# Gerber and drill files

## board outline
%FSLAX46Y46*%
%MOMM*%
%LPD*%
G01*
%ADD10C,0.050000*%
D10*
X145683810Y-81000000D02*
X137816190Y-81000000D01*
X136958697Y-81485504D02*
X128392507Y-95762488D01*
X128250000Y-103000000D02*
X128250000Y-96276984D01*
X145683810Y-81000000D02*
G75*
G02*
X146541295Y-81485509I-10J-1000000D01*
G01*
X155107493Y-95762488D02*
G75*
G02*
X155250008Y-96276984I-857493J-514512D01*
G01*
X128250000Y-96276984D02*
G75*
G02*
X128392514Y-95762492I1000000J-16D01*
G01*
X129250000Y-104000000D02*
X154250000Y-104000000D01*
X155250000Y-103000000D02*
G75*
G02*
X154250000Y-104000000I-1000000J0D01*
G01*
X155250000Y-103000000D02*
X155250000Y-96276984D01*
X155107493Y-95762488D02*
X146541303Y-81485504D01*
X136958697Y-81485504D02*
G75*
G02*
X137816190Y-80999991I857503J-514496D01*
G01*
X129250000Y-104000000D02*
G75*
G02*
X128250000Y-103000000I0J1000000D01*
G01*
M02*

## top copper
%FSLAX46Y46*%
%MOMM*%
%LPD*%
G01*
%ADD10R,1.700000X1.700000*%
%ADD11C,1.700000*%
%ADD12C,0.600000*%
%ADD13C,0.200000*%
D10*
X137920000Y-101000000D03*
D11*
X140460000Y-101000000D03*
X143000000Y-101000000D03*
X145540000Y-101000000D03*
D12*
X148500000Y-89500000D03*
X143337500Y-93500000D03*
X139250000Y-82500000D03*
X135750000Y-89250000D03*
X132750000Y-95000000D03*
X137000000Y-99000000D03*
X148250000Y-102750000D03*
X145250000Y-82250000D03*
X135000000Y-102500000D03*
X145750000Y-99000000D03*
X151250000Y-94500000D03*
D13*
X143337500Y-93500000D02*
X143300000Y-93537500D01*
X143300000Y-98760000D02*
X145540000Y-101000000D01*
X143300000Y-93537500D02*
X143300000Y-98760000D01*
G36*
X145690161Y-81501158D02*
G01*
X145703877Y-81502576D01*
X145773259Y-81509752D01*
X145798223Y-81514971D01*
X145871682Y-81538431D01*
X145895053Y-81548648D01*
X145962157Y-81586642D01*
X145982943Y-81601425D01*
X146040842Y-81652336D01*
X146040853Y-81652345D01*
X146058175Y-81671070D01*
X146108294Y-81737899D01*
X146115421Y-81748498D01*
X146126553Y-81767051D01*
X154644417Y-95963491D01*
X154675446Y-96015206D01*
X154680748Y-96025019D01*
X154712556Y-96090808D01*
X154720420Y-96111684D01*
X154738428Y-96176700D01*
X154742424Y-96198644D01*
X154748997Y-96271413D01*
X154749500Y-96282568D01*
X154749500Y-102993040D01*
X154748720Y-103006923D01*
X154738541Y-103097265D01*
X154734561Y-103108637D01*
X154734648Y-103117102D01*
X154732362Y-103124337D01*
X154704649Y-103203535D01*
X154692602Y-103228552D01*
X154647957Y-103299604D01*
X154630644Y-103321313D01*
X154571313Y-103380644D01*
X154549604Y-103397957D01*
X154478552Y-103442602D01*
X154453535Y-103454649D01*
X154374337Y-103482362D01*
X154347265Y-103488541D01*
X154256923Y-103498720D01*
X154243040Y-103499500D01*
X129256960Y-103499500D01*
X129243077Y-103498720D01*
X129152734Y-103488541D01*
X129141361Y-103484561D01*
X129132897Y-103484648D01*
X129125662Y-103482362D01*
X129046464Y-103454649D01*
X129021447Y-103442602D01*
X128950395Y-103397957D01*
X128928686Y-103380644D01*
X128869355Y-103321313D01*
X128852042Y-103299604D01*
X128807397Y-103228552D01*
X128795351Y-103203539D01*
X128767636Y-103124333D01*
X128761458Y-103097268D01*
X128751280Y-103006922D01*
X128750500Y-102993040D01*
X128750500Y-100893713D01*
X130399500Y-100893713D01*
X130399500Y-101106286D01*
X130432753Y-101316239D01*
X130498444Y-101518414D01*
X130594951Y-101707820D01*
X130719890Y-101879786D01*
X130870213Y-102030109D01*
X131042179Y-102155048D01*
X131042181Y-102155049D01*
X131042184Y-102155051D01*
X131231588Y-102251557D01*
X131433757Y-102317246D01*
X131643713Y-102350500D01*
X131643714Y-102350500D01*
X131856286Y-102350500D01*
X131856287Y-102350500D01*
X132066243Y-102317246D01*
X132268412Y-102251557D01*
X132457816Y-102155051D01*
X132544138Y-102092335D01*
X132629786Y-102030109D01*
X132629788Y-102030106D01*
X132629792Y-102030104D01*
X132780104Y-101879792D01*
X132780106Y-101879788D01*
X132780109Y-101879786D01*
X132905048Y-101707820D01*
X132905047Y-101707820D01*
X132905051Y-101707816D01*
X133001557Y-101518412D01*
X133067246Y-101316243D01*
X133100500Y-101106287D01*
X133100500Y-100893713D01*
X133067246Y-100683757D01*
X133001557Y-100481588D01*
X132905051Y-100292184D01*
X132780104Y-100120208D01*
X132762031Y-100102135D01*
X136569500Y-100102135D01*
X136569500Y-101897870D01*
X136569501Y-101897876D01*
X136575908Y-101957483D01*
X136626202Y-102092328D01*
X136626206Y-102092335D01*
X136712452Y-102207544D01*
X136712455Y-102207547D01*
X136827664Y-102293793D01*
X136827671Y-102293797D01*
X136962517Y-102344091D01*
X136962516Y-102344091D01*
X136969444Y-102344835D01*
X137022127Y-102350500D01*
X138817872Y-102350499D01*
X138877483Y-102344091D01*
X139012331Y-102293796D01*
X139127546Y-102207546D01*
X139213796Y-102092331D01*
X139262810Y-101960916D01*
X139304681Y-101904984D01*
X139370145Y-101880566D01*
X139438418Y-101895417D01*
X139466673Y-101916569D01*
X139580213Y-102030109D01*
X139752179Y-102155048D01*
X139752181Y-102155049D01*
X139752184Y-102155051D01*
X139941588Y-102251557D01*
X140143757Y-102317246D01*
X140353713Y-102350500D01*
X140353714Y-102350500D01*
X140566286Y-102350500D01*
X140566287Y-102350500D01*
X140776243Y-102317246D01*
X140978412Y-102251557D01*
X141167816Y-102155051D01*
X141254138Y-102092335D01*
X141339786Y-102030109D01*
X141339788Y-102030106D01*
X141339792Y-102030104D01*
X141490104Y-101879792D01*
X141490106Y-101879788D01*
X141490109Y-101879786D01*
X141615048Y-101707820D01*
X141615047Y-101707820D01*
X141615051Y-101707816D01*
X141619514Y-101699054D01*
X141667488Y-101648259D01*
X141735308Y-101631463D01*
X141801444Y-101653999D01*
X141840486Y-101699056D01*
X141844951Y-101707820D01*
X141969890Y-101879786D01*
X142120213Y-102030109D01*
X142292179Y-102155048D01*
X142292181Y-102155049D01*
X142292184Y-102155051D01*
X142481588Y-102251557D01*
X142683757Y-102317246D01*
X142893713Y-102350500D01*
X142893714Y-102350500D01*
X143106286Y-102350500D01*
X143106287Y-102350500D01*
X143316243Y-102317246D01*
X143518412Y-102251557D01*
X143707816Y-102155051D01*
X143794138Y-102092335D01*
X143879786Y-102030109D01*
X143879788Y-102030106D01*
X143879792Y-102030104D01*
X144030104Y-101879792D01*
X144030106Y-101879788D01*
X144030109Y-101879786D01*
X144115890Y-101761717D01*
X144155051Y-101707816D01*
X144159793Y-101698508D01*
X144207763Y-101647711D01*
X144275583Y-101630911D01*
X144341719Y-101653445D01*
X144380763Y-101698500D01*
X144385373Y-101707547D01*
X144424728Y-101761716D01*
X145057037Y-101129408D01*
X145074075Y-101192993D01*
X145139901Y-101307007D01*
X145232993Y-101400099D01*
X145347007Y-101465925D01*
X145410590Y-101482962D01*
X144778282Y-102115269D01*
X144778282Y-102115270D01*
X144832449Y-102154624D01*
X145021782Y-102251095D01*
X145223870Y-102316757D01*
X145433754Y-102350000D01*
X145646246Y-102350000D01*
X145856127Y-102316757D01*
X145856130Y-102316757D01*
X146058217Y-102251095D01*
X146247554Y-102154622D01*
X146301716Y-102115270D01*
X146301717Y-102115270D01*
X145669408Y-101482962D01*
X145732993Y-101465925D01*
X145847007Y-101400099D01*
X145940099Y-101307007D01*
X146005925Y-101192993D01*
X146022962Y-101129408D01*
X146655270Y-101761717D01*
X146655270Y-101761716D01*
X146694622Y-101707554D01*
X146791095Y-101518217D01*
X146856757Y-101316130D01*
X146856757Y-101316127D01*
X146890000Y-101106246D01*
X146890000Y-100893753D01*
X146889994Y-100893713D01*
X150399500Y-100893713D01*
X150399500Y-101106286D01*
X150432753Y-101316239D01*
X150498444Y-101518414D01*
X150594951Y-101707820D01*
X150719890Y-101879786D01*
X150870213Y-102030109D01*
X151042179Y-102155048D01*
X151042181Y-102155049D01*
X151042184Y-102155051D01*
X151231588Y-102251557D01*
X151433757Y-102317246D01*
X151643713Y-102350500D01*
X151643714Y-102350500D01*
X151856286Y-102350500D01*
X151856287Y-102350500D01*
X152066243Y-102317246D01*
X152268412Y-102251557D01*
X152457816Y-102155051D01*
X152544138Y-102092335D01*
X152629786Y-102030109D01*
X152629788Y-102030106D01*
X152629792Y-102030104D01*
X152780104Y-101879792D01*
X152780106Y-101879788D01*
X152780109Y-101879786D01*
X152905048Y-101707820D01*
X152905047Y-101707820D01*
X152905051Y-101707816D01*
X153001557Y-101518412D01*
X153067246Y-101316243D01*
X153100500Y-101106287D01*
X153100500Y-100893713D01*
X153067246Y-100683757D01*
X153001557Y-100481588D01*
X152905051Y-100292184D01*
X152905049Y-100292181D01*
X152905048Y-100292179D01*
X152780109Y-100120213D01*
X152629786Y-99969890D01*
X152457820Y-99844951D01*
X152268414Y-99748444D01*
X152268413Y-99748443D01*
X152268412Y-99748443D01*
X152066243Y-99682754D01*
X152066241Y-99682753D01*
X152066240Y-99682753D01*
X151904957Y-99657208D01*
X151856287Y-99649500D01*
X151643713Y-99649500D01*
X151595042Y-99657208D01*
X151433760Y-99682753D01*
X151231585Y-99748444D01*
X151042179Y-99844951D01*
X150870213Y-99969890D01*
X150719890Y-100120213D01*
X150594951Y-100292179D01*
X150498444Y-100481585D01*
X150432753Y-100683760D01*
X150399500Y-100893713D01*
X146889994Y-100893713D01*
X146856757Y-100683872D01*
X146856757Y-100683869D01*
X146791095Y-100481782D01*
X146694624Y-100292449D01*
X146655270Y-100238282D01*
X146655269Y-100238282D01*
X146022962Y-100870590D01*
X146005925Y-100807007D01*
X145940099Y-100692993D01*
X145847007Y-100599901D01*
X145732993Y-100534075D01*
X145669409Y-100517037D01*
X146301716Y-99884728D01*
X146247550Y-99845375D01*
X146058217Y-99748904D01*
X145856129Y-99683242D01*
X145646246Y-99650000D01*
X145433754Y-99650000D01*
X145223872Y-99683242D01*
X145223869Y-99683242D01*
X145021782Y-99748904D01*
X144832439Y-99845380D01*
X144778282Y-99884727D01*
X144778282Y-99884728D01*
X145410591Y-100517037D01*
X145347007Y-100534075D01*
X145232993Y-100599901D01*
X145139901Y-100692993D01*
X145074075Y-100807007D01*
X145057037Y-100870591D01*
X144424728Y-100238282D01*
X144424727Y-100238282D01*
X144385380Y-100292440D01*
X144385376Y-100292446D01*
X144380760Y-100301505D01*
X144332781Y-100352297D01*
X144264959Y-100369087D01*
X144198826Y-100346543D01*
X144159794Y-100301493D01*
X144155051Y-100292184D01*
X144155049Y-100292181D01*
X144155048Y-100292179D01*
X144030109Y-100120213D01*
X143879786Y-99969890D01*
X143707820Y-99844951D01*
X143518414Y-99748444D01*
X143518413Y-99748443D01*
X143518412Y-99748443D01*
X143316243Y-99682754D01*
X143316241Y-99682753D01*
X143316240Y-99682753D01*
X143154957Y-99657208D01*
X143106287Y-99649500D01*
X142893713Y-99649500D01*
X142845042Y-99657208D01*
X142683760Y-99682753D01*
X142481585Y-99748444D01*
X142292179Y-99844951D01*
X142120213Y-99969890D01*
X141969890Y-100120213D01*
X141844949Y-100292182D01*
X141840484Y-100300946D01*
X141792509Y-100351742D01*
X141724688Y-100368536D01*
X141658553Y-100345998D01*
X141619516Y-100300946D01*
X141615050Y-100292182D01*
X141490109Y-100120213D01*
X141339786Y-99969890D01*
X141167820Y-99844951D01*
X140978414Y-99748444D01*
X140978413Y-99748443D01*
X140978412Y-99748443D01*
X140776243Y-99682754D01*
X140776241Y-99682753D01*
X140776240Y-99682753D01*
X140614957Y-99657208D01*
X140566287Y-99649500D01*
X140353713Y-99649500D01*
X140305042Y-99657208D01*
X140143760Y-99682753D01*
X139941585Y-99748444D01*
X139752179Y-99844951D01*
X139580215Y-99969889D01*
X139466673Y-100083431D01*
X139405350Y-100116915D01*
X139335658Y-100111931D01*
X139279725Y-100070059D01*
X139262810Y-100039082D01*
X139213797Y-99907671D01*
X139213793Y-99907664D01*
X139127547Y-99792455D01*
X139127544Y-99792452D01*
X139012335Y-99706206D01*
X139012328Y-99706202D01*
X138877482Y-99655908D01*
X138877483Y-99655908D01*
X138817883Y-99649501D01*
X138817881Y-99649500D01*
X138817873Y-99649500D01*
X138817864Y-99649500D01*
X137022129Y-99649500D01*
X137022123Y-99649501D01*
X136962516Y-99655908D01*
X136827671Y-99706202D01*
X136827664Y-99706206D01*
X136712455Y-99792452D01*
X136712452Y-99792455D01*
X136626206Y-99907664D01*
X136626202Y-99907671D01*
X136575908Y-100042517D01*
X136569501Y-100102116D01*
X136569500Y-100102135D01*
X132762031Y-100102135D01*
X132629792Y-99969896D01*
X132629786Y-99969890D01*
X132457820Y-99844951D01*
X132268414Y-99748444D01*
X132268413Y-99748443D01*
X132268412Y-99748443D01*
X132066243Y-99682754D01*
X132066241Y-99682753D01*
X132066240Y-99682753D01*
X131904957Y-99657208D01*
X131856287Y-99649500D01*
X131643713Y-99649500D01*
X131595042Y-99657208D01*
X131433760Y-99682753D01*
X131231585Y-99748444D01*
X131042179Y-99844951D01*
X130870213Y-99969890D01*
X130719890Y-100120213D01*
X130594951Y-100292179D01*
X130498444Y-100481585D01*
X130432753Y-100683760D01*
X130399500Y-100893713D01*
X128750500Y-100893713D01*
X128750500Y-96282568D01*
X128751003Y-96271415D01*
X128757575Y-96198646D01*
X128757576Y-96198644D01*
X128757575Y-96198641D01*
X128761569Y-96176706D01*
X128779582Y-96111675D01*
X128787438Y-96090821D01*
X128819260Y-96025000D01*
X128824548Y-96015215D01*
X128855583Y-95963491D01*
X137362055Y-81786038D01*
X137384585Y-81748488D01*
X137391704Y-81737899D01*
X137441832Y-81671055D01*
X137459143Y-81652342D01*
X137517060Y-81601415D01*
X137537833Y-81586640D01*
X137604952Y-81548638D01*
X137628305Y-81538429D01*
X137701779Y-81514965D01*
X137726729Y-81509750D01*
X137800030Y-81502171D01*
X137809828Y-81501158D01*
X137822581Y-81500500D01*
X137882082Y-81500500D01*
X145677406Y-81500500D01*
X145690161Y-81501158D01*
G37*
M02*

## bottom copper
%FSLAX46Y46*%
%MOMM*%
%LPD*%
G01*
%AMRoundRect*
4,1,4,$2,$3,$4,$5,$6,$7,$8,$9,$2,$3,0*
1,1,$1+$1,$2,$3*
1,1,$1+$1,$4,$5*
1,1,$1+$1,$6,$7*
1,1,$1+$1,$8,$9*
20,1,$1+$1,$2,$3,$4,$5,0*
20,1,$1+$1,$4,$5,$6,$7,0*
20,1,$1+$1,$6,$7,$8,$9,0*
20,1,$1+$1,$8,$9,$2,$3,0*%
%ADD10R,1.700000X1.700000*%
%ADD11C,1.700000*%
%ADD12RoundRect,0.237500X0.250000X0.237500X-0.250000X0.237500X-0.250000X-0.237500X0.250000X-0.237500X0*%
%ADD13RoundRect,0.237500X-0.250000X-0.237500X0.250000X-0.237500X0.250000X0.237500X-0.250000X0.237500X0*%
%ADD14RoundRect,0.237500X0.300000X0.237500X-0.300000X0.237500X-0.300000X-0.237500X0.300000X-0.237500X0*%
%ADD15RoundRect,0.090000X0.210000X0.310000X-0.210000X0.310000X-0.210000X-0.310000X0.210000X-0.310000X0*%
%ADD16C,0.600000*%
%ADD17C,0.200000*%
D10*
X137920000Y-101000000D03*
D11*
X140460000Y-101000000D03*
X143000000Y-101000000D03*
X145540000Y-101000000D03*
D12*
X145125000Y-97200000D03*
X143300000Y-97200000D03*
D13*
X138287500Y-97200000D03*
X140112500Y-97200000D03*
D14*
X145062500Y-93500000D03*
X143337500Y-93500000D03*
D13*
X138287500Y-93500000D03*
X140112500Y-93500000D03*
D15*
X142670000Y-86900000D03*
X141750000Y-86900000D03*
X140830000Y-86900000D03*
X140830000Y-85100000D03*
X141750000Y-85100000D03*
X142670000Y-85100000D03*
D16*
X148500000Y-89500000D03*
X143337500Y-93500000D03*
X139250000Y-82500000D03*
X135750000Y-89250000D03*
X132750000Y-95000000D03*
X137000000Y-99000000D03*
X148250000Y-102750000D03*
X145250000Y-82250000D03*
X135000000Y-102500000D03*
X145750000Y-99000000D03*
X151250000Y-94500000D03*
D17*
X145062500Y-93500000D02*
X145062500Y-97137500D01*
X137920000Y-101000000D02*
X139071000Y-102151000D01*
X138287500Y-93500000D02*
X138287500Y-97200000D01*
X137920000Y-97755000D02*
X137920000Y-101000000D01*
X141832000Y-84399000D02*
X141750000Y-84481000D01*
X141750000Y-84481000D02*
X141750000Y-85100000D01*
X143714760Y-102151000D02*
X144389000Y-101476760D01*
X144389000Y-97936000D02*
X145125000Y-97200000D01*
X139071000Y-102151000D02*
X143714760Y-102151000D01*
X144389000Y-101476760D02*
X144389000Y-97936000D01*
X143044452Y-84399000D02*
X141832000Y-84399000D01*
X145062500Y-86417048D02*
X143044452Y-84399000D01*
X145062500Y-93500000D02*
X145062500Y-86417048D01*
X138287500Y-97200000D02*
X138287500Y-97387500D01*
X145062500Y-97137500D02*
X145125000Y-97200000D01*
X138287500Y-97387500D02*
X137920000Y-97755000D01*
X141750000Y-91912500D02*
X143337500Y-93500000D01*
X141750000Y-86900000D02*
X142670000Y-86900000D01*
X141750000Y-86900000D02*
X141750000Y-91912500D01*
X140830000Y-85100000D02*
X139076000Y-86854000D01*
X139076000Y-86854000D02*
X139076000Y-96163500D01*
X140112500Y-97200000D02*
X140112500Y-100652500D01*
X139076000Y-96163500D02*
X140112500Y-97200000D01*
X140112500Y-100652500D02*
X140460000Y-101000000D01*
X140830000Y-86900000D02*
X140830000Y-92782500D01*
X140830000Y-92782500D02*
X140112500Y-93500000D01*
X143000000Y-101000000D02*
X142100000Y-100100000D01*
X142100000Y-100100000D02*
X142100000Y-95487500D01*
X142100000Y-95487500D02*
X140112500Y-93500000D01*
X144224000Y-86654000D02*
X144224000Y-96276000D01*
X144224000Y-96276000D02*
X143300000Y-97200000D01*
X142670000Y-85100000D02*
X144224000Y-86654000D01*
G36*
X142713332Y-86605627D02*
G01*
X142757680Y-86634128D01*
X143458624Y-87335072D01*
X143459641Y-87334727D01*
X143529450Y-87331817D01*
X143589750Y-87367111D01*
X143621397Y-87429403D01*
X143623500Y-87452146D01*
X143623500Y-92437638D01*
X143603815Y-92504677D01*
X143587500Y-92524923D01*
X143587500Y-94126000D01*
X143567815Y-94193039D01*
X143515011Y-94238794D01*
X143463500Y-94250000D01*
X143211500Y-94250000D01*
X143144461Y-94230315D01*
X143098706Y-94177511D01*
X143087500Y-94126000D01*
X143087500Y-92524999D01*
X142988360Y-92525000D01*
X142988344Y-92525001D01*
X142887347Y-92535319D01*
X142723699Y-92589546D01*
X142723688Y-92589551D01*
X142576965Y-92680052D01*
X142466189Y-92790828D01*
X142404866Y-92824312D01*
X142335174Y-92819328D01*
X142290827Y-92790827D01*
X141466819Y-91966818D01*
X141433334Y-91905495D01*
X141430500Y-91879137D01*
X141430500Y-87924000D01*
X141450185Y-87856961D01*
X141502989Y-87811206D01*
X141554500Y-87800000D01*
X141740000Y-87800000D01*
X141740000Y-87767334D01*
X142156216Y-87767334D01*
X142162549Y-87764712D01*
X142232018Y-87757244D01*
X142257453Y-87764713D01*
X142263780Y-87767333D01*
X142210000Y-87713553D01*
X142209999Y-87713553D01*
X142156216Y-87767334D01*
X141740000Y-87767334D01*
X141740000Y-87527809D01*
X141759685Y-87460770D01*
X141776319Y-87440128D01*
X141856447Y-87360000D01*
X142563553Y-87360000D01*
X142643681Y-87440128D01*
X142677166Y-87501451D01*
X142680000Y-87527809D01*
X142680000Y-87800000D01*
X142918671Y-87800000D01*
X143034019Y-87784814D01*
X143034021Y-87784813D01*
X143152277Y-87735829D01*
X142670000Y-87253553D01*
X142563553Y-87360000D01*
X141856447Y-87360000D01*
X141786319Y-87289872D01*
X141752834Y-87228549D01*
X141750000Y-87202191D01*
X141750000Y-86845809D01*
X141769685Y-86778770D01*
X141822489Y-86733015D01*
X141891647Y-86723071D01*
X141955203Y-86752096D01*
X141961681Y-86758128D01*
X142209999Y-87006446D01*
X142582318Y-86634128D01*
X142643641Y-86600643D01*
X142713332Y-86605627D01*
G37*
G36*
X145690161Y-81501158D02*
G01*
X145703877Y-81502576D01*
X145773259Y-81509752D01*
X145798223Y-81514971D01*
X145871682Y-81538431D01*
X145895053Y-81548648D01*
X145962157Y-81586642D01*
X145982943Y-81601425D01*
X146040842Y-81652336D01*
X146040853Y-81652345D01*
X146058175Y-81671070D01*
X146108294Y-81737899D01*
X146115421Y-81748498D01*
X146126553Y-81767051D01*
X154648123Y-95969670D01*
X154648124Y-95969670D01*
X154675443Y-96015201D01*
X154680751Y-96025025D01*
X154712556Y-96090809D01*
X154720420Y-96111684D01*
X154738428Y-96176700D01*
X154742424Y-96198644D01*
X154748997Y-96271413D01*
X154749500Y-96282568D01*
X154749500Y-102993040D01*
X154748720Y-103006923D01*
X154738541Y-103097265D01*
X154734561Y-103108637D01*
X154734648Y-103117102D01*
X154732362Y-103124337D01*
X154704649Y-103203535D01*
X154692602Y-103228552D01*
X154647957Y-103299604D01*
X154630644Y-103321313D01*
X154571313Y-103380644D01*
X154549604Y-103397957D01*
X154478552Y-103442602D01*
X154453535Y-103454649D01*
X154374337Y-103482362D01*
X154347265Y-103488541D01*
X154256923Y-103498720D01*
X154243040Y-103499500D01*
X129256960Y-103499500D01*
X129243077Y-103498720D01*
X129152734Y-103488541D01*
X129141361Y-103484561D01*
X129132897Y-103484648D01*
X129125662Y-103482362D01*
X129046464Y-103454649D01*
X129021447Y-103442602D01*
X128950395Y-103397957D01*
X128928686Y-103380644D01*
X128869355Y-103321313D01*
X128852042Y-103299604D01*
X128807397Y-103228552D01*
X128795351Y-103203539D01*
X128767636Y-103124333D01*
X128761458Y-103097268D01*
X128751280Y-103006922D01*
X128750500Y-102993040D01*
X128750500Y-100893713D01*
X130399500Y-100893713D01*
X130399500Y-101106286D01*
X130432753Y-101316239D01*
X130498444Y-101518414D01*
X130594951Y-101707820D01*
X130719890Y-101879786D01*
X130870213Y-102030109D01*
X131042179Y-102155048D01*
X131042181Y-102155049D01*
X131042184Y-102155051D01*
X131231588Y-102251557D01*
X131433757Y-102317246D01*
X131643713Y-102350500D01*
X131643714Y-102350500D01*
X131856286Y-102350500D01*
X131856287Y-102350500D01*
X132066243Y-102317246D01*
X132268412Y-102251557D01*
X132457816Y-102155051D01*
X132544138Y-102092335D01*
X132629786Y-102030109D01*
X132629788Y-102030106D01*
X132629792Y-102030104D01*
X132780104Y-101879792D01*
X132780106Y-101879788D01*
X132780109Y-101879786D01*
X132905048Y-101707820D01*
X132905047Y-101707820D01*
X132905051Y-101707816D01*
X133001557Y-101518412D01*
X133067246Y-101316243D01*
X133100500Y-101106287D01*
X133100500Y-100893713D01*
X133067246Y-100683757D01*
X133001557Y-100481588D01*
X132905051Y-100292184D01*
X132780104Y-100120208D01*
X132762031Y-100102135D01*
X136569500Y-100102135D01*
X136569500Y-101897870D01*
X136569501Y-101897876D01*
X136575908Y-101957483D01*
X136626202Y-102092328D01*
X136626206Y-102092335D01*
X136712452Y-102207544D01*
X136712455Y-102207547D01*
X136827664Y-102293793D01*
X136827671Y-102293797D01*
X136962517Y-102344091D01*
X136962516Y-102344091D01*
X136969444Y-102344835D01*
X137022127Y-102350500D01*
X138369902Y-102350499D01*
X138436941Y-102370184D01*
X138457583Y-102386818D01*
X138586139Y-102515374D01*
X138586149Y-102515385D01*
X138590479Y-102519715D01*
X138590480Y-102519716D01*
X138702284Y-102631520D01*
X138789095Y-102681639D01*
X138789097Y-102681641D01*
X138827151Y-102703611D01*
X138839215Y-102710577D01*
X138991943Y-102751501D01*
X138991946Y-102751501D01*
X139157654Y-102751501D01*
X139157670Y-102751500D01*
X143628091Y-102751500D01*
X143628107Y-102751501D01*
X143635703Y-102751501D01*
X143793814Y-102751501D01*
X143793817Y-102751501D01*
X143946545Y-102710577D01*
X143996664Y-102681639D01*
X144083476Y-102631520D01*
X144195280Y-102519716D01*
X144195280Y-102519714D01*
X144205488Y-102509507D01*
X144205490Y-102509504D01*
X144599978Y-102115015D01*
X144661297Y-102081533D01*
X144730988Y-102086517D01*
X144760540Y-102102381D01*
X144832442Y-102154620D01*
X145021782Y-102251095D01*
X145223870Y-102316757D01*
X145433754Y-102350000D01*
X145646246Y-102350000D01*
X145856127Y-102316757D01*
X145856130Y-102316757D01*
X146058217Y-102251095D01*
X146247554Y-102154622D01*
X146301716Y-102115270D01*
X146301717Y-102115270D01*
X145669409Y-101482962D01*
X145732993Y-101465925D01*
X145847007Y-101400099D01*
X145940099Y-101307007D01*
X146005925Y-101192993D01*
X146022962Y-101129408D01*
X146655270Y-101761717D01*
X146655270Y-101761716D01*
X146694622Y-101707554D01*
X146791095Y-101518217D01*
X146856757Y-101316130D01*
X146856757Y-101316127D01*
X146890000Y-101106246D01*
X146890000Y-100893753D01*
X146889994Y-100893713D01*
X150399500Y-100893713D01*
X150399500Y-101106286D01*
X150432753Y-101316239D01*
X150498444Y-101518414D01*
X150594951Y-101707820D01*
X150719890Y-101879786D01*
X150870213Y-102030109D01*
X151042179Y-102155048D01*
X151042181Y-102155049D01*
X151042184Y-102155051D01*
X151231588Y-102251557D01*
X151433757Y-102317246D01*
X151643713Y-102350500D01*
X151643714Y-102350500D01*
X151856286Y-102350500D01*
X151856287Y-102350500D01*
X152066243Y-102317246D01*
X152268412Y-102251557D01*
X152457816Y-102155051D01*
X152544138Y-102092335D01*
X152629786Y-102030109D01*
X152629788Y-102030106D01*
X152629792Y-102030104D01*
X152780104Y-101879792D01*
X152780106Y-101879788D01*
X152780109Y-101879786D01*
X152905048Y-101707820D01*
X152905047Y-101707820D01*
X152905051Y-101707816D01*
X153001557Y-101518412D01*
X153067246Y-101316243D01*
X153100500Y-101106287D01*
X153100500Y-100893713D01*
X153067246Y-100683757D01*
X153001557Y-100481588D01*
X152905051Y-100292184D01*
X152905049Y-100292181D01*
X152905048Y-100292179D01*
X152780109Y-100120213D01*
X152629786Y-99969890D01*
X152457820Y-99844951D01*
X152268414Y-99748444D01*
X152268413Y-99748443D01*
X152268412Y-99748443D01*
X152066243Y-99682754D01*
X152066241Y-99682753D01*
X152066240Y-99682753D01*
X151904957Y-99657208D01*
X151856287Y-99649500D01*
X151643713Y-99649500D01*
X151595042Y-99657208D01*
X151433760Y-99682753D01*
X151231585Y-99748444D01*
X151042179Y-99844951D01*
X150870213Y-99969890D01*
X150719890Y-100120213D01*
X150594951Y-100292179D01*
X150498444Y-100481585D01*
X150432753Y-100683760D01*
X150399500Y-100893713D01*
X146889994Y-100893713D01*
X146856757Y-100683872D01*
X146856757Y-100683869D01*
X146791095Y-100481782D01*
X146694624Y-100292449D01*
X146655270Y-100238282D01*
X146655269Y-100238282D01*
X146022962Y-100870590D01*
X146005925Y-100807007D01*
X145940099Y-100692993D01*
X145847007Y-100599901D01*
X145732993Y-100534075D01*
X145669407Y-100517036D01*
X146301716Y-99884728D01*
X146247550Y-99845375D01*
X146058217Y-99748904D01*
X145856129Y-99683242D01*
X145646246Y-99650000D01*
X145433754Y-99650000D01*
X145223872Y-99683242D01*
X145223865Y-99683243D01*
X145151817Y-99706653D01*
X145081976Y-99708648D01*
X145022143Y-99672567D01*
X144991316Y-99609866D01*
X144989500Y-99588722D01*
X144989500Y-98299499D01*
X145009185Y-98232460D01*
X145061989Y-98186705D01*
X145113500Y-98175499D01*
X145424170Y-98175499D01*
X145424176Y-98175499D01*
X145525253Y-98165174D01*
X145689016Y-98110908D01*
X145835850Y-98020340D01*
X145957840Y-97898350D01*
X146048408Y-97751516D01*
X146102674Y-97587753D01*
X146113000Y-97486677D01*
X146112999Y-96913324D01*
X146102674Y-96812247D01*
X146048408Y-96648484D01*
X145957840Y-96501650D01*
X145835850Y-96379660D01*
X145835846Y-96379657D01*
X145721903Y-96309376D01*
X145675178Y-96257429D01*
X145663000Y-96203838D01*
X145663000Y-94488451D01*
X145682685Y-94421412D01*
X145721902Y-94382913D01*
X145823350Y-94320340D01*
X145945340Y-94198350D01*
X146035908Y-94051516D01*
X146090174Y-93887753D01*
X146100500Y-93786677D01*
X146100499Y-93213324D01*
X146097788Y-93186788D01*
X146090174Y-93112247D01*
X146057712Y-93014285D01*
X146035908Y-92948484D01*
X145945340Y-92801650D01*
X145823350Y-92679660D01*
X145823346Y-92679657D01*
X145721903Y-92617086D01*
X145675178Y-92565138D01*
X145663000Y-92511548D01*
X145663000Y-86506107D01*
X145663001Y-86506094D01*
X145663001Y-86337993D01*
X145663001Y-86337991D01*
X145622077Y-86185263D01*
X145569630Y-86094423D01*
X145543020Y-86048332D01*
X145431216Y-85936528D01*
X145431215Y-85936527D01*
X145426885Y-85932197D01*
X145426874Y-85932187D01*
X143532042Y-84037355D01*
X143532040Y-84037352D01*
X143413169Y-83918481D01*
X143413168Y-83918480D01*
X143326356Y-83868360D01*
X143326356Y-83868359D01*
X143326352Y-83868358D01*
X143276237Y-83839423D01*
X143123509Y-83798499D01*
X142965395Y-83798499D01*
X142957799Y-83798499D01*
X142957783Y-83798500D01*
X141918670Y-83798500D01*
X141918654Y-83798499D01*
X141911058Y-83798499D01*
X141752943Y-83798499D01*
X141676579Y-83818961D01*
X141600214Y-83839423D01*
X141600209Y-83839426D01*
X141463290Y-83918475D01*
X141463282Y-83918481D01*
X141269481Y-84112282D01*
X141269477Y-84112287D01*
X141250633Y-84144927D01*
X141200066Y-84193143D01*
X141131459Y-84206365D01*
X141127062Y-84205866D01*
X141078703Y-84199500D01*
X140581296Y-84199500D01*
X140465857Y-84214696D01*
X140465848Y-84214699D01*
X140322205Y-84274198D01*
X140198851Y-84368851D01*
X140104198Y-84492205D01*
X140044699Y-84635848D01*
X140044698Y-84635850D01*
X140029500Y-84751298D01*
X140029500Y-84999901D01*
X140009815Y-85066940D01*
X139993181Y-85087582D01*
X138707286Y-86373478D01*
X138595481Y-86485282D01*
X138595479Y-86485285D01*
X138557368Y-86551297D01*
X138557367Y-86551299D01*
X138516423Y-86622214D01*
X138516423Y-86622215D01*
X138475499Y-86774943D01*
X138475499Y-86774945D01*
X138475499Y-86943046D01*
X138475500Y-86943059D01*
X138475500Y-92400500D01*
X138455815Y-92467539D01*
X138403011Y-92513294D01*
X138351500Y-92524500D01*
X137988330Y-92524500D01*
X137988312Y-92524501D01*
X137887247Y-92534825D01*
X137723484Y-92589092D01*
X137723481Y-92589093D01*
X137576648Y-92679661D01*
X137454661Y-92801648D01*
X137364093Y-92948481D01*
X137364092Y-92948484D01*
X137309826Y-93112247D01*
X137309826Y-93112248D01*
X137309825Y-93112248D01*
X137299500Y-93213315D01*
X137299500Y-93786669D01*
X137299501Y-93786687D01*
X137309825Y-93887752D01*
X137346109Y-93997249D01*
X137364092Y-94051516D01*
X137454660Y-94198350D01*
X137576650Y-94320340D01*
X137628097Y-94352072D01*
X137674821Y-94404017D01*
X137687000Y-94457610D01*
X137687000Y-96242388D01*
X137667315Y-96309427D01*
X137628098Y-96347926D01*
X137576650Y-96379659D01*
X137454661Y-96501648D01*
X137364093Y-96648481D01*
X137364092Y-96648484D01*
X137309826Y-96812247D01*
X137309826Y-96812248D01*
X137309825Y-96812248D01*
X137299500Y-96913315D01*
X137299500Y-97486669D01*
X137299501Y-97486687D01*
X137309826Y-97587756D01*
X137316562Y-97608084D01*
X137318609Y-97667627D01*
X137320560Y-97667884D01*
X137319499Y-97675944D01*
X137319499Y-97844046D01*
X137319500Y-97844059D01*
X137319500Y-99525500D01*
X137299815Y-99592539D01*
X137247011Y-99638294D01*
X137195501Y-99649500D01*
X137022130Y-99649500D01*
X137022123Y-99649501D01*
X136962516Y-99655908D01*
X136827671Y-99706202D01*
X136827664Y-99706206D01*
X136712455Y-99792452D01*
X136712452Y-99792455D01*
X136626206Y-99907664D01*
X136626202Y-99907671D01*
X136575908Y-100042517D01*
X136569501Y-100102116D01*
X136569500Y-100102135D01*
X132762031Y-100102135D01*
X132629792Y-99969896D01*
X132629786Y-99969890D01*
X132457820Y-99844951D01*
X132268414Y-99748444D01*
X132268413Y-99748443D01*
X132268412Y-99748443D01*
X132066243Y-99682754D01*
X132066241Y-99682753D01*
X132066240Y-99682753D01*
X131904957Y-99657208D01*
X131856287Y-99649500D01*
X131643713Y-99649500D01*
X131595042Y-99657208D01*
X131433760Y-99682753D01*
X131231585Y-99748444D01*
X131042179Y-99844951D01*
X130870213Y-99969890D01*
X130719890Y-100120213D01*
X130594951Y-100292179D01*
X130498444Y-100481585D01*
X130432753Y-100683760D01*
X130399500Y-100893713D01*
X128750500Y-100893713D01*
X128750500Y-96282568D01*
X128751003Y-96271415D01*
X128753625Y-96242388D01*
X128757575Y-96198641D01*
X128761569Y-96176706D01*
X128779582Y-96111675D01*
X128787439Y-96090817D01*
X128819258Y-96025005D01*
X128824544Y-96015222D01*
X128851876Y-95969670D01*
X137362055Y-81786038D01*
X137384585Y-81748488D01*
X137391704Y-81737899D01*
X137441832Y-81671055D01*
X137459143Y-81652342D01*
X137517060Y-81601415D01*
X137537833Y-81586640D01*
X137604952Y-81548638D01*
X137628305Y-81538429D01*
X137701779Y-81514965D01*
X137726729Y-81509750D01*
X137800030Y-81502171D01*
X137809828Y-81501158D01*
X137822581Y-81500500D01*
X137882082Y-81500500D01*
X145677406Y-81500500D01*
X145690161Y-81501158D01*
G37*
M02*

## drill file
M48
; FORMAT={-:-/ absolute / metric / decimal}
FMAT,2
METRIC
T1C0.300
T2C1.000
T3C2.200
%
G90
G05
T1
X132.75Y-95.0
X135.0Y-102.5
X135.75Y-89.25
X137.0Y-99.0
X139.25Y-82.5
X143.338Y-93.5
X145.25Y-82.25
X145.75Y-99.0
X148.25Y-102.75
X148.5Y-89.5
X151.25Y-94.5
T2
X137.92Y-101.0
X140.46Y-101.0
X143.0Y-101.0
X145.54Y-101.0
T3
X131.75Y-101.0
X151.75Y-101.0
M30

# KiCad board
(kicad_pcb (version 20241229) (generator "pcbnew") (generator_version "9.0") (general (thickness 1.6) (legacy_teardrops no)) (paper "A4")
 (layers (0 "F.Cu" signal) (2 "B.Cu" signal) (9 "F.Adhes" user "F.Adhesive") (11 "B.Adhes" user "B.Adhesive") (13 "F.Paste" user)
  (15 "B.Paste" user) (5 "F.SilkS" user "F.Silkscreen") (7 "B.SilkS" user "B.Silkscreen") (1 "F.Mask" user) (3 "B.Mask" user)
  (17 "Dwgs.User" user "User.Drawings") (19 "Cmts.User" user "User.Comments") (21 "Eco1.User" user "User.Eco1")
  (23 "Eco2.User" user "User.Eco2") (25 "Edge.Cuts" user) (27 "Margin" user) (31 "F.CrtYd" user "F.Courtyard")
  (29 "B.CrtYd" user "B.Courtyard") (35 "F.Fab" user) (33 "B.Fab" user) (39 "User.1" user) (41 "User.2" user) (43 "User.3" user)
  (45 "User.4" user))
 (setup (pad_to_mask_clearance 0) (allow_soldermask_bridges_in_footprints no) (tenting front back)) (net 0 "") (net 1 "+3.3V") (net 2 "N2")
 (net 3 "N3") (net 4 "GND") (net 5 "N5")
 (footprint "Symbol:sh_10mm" (layer "F.Cu") (at 141.75 92.25)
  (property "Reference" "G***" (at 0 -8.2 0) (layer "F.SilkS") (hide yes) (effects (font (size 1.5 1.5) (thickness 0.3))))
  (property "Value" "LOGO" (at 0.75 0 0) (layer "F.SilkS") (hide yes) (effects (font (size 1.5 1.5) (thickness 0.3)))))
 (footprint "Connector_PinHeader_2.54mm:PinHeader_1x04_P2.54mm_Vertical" (layer "F.Cu") (at 137.92 101 90)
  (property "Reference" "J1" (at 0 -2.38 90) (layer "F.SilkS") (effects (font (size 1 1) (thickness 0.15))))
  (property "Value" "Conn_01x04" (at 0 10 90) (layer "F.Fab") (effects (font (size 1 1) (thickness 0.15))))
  (pad "1" thru_hole rect (at 0 0 90) (size 1.7 1.7) (drill 1) (layers "*.Cu" "*.Mask") (remove_unused_layers no) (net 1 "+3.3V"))
  (pad "2" thru_hole circle (at 0 2.54 90) (size 1.7 1.7) (drill 1) (layers "*.Cu" "*.Mask") (remove_unused_layers no) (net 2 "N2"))
  (pad "3" thru_hole circle (at 0 5.08 90) (size 1.7 1.7) (drill 1) (layers "*.Cu" "*.Mask") (remove_unused_layers no) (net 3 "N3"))
  (pad "4" thru_hole circle (at 0 7.62 90) (size 1.7 1.7) (drill 1) (layers "*.Cu" "*.Mask") (remove_unused_layers no) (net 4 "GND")))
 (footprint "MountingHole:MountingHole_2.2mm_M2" (layer "F.Cu") (at 131.75 101)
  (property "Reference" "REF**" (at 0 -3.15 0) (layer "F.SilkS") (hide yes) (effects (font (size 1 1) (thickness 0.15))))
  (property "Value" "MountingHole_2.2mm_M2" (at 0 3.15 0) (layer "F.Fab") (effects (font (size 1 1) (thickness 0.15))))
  (pad "" np_thru_hole circle (at 0 0) (size 2.2 2.2) (drill 2.2) (layers "*.Cu" "*.Mask")))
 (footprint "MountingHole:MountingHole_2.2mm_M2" (layer "F.Cu") (at 151.75 101)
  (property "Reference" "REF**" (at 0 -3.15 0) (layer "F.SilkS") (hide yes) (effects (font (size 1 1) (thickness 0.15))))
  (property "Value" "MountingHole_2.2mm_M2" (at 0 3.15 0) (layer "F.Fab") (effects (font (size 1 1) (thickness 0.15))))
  (pad "" np_thru_hole circle (at 0 0) (size 2.2 2.2) (drill 2.2) (layers "*.Cu" "*.Mask")))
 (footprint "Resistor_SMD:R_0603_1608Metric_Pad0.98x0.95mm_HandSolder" (layer "B.Cu") (at 144.2125 97.2 180)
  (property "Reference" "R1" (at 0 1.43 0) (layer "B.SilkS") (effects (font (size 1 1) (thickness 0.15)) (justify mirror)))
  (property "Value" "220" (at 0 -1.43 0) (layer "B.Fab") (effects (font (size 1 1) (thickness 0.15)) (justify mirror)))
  (pad "1" smd roundrect (at -0.9125 0 180) (size 0.975 0.95) (layers "B.Cu" "B.Mask" "B.Paste") (roundrect_rratio 0.25) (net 1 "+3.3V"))
  (pad "2" smd roundrect (at 0.9125 0 180) (size 0.975 0.95) (layers "B.Cu" "B.Mask" "B.Paste") (roundrect_rratio 0.25) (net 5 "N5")))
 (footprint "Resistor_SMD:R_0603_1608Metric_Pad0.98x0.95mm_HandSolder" (layer "B.Cu") (at 139.2 97.2)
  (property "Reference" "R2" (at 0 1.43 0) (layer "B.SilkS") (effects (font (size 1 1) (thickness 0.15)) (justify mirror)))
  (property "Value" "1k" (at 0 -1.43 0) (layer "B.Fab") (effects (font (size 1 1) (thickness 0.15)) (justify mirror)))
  (pad "1" smd roundrect (at -0.9125 0) (size 0.975 0.95) (layers "B.Cu" "B.Mask" "B.Paste") (roundrect_rratio 0.25) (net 1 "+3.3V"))
  (pad "2" smd roundrect (at 0.9125 0) (size 0.975 0.95) (layers "B.Cu" "B.Mask" "B.Paste") (roundrect_rratio 0.25) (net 2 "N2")))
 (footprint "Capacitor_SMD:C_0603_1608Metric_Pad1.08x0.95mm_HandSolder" (layer "B.Cu") (at 144.2 93.5 180)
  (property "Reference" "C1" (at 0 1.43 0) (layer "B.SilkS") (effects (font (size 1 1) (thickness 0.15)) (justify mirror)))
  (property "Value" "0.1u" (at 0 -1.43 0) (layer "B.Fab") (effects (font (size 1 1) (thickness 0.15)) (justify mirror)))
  (pad "1" smd roundrect (at -0.8625 0 180) (size 1.075 0.95) (layers "B.Cu" "B.Mask" "B.Paste") (roundrect_rratio 0.25) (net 1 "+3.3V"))
  (pad "2" smd roundrect (at 0.8625 0 180) (size 1.075 0.95) (layers "B.Cu" "B.Mask" "B.Paste") (roundrect_rratio 0.25) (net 4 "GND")))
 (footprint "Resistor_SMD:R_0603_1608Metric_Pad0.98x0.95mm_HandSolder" (layer "B.Cu") (at 139.2 93.5)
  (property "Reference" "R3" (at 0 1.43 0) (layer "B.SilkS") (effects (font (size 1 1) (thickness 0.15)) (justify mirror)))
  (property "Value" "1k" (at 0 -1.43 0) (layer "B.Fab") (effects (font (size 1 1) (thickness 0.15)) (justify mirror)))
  (pad "1" smd roundrect (at -0.9125 0) (size 0.975 0.95) (layers "B.Cu" "B.Mask" "B.Paste") (roundrect_rratio 0.25) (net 1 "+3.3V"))
  (pad "2" smd roundrect (at 0.9125 0) (size 0.975 0.95) (layers "B.Cu" "B.Mask" "B.Paste") (roundrect_rratio 0.25) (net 3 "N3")))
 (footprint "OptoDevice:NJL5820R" (layer "B.Cu") (at 141.75 86 180)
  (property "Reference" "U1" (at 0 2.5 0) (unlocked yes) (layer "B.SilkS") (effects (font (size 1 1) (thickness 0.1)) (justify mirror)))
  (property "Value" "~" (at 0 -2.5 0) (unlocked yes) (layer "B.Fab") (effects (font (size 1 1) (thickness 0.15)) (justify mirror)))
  (pad "1" smd roundrect (at -0.92 -0.9 180) (size 0.6 0.8) (layers "B.Cu" "B.Mask" "B.Paste") (roundrect_rratio 0.15) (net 4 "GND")
   (thermal_bridge_angle 45))
  (pad "2" smd roundrect (at 0 -0.9 180) (size 0.6 0.8) (layers "B.Cu" "B.Mask" "B.Paste") (roundrect_rratio 0.15) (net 4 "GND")
   (thermal_bridge_angle 45))
  (pad "3" smd roundrect (at 0.92 -0.9 180) (size 0.6 0.8) (layers "B.Cu" "B.Mask" "B.Paste") (roundrect_rratio 0.15) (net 3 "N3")
   (thermal_bridge_angle 45))
  (pad "4" smd roundrect (at 0.92 0.9 180) (size 0.6 0.8) (layers "B.Cu" "B.Mask" "B.Paste") (roundrect_rratio 0.15) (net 2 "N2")
   (thermal_bridge_angle 45))
  (pad "5" smd roundrect (at 0 0.9 180) (size 0.6 0.8) (layers "B.Cu" "B.Mask" "B.Paste") (roundrect_rratio 0.15) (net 1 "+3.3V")
   (thermal_bridge_angle 45))
  (pad "6" smd roundrect (at -0.92 0.9 180) (size 0.6 0.8) (layers "B.Cu" "B.Mask" "B.Paste") (roundrect_rratio 0.15) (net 5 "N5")
   (thermal_bridge_angle 45)))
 (gr_line (start 145.68381 81) (end 137.81619 81) (stroke (width 0.05) (type default)) (layer "Edge.Cuts"))
 (gr_line (start 136.958697 81.485504) (end 128.392507 95.762488) (stroke (width 0.05) (type default)) (layer "Edge.Cuts"))
 (gr_line (start 128.25 103) (end 128.25 96.276984) (stroke (width 0.05) (type default)) (layer "Edge.Cuts"))
 (gr_arc (start 145.68381 81) (mid 146.176505 81.129804) (end 146.541303 81.485504) (stroke (width 0.05) (type default)) (layer "Edge.Cuts"))
 (gr_arc (start 155.107493 95.762488) (mid 155.213715 96.01005) (end 155.25 96.276984) (stroke (width 0.05) (type default))
  (layer "Edge.Cuts"))
 (gr_arc (start 128.25 96.276984) (mid 128.286285 96.01005) (end 128.392507 95.762488) (stroke (width 0.05) (type default))
  (layer "Edge.Cuts"))
 (gr_line (start 129.25 104) (end 154.25 104) (stroke (width 0.05) (type default)) (layer "Edge.Cuts"))
 (gr_arc (start 155.25 103) (mid 154.957107 103.707107) (end 154.25 104) (stroke (width 0.05) (type default)) (layer "Edge.Cuts"))
 (gr_line (start 155.25 103) (end 155.25 96.276984) (stroke (width 0.05) (type default)) (layer "Edge.Cuts"))
 (gr_line (start 155.107493 95.762488) (end 146.541303 81.485504) (stroke (width 0.05) (type default)) (layer "Edge.Cuts"))
 (gr_arc (start 136.958697 81.485504) (mid 137.323491 81.1298) (end 137.81619 81) (stroke (width 0.05) (type default)) (layer "Edge.Cuts"))
 (gr_arc (start 129.25 104) (mid 128.542893 103.707107) (end 128.25 103) (stroke (width 0.05) (type default)) (layer "Edge.Cuts"))
 (segment (start 145.0625 93.5) (end 145.0625 97.1375) (width 0.2) (layer "B.Cu") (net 1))
 (segment (start 137.92 101) (end 139.071 102.151) (width 0.2) (layer "B.Cu") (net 1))
 (segment (start 138.2875 93.5) (end 138.2875 97.2) (width 0.2) (layer "B.Cu") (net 1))
 (segment (start 137.92 97.755) (end 137.92 101) (width 0.2) (layer "B.Cu") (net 1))
 (segment (start 141.832 84.399) (end 141.75 84.481) (width 0.2) (layer "B.Cu") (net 1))
 (segment (start 141.75 84.481) (end 141.75 85.1) (width 0.2) (layer "B.Cu") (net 1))
 (segment (start 143.71476 102.151) (end 144.389 101.47676) (width 0.2) (layer "B.Cu") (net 1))
 (segment (start 144.389 97.936) (end 145.125 97.2) (width 0.2) (layer "B.Cu") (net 1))
 (segment (start 139.071 102.151) (end 143.71476 102.151) (width 0.2) (layer "B.Cu") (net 1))
 (segment (start 144.389 101.47676) (end 144.389 97.936) (width 0.2) (layer "B.Cu") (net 1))
 (segment (start 143.044452 84.399) (end 141.832 84.399) (width 0.2) (layer "B.Cu") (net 1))
 (segment (start 145.0625 86.417048) (end 143.044452 84.399) (width 0.2) (layer "B.Cu") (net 1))
 (segment (start 145.0625 93.5) (end 145.0625 86.417048) (width 0.2) (layer "B.Cu") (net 1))
 (segment (start 138.2875 97.2) (end 138.2875 97.3875) (width 0.2) (layer "B.Cu") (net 1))
 (segment (start 145.0625 97.1375) (end 145.125 97.2) (width 0.2) (layer "B.Cu") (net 1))
 (segment (start 138.2875 97.3875) (end 137.92 97.755) (width 0.2) (layer "B.Cu") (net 1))
 (segment (start 143.3375 93.5) (end 143.3 93.5375) (width 0.2) (layer "F.Cu") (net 4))
 (segment (start 143.3 98.76) (end 145.54 101) (width 0.2) (layer "F.Cu") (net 4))
 (segment (start 143.3 93.5375) (end 143.3 98.76) (width 0.2) (layer "F.Cu") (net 4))
 (via (at 148.5 89.5) (size 0.6) (drill 0.3) (layers "F.Cu" "B.Cu") (free yes) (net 4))
 (via (at 143.3375 93.5) (size 0.6) (drill 0.3) (layers "F.Cu" "B.Cu") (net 4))
 (via (at 139.25 82.5) (size 0.6) (drill 0.3) (layers "F.Cu" "B.Cu") (free yes) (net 4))
 (via (at 135.75 89.25) (size 0.6) (drill 0.3) (layers "F.Cu" "B.Cu") (free yes) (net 4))
 (via (at 132.75 95) (size 0.6) (drill 0.3) (layers "F.Cu" "B.Cu") (free yes) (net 4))
 (via (at 137 99) (size 0.6) (drill 0.3) (layers "F.Cu" "B.Cu") (free yes) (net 4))
 (via (at 148.25 102.75) (size 0.6) (drill 0.3) (layers "F.Cu" "B.Cu") (free yes) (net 4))
 (via (at 145.25 82.25) (size 0.6) (drill 0.3) (layers "F.Cu" "B.Cu") (free yes) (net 4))
 (via (at 135 102.5) (size 0.6) (drill 0.3) (layers "F.Cu" "B.Cu") (free yes) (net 4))
 (via (at 145.75 99) (size 0.6) (drill 0.3) (layers "F.Cu" "B.Cu") (free yes) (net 4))
 (via (at 151.25 94.5) (size 0.6) (drill 0.3) (layers "F.Cu" "B.Cu") (free yes) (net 4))
 (segment (start 141.75 91.9125) (end 143.3375 93.5) (width 0.2) (layer "B.Cu") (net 4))
 (segment (start 141.75 86.9) (end 142.67 86.9) (width 0.2) (layer "B.Cu") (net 4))
 (segment (start 141.75 86.9) (end 141.75 91.9125) (width 0.2) (layer "B.Cu") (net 4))
 (segment (start 140.83 85.1) (end 139.076 86.854) (width 0.2) (layer "B.Cu") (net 2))
 (segment (start 139.076 86.854) (end 139.076 96.1635) (width 0.2) (layer "B.Cu") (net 2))
 (segment (start 140.1125 97.2) (end 140.1125 100.6525) (width 0.2) (layer "B.Cu") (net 2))
 (segment (start 139.076 96.1635) (end 140.1125 97.2) (width 0.2) (layer "B.Cu") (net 2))
 (segment (start 140.1125 100.6525) (end 140.46 101) (width 0.2) (layer "B.Cu") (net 2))
 (segment (start 140.83 86.9) (end 140.83 92.7825) (width 0.2) (layer "B.Cu") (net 3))
 (segment (start 140.83 92.7825) (end 140.1125 93.5) (width 0.2) (layer "B.Cu") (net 3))
 (segment (start 143 101) (end 142.1 100.1) (width 0.2) (layer "B.Cu") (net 3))
 (segment (start 142.1 100.1) (end 142.1 95.4875) (width 0.2) (layer "B.Cu") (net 3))
 (segment (start 142.1 95.4875) (end 140.1125 93.5) (width 0.2) (layer "B.Cu") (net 3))
 (segment (start 144.224 86.654) (end 144.224 96.276) (width 0.2) (layer "B.Cu") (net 5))
 (segment (start 144.224 96.276) (end 143.3 97.2) (width 0.2) (layer "B.Cu") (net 5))
 (segment (start 142.67 85.1) (end 144.224 86.654) (width 0.2) (layer "B.Cu") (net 5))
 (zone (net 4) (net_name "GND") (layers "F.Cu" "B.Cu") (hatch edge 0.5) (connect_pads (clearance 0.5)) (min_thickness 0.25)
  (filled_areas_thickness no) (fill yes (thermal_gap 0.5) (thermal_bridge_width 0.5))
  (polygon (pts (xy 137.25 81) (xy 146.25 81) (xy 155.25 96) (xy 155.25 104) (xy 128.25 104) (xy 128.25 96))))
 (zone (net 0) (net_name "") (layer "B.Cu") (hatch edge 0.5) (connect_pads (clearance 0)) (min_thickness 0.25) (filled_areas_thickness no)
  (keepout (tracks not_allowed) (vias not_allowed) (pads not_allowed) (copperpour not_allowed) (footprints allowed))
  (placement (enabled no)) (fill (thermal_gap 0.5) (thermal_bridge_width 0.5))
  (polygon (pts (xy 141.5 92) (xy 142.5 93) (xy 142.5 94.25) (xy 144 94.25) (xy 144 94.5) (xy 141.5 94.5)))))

